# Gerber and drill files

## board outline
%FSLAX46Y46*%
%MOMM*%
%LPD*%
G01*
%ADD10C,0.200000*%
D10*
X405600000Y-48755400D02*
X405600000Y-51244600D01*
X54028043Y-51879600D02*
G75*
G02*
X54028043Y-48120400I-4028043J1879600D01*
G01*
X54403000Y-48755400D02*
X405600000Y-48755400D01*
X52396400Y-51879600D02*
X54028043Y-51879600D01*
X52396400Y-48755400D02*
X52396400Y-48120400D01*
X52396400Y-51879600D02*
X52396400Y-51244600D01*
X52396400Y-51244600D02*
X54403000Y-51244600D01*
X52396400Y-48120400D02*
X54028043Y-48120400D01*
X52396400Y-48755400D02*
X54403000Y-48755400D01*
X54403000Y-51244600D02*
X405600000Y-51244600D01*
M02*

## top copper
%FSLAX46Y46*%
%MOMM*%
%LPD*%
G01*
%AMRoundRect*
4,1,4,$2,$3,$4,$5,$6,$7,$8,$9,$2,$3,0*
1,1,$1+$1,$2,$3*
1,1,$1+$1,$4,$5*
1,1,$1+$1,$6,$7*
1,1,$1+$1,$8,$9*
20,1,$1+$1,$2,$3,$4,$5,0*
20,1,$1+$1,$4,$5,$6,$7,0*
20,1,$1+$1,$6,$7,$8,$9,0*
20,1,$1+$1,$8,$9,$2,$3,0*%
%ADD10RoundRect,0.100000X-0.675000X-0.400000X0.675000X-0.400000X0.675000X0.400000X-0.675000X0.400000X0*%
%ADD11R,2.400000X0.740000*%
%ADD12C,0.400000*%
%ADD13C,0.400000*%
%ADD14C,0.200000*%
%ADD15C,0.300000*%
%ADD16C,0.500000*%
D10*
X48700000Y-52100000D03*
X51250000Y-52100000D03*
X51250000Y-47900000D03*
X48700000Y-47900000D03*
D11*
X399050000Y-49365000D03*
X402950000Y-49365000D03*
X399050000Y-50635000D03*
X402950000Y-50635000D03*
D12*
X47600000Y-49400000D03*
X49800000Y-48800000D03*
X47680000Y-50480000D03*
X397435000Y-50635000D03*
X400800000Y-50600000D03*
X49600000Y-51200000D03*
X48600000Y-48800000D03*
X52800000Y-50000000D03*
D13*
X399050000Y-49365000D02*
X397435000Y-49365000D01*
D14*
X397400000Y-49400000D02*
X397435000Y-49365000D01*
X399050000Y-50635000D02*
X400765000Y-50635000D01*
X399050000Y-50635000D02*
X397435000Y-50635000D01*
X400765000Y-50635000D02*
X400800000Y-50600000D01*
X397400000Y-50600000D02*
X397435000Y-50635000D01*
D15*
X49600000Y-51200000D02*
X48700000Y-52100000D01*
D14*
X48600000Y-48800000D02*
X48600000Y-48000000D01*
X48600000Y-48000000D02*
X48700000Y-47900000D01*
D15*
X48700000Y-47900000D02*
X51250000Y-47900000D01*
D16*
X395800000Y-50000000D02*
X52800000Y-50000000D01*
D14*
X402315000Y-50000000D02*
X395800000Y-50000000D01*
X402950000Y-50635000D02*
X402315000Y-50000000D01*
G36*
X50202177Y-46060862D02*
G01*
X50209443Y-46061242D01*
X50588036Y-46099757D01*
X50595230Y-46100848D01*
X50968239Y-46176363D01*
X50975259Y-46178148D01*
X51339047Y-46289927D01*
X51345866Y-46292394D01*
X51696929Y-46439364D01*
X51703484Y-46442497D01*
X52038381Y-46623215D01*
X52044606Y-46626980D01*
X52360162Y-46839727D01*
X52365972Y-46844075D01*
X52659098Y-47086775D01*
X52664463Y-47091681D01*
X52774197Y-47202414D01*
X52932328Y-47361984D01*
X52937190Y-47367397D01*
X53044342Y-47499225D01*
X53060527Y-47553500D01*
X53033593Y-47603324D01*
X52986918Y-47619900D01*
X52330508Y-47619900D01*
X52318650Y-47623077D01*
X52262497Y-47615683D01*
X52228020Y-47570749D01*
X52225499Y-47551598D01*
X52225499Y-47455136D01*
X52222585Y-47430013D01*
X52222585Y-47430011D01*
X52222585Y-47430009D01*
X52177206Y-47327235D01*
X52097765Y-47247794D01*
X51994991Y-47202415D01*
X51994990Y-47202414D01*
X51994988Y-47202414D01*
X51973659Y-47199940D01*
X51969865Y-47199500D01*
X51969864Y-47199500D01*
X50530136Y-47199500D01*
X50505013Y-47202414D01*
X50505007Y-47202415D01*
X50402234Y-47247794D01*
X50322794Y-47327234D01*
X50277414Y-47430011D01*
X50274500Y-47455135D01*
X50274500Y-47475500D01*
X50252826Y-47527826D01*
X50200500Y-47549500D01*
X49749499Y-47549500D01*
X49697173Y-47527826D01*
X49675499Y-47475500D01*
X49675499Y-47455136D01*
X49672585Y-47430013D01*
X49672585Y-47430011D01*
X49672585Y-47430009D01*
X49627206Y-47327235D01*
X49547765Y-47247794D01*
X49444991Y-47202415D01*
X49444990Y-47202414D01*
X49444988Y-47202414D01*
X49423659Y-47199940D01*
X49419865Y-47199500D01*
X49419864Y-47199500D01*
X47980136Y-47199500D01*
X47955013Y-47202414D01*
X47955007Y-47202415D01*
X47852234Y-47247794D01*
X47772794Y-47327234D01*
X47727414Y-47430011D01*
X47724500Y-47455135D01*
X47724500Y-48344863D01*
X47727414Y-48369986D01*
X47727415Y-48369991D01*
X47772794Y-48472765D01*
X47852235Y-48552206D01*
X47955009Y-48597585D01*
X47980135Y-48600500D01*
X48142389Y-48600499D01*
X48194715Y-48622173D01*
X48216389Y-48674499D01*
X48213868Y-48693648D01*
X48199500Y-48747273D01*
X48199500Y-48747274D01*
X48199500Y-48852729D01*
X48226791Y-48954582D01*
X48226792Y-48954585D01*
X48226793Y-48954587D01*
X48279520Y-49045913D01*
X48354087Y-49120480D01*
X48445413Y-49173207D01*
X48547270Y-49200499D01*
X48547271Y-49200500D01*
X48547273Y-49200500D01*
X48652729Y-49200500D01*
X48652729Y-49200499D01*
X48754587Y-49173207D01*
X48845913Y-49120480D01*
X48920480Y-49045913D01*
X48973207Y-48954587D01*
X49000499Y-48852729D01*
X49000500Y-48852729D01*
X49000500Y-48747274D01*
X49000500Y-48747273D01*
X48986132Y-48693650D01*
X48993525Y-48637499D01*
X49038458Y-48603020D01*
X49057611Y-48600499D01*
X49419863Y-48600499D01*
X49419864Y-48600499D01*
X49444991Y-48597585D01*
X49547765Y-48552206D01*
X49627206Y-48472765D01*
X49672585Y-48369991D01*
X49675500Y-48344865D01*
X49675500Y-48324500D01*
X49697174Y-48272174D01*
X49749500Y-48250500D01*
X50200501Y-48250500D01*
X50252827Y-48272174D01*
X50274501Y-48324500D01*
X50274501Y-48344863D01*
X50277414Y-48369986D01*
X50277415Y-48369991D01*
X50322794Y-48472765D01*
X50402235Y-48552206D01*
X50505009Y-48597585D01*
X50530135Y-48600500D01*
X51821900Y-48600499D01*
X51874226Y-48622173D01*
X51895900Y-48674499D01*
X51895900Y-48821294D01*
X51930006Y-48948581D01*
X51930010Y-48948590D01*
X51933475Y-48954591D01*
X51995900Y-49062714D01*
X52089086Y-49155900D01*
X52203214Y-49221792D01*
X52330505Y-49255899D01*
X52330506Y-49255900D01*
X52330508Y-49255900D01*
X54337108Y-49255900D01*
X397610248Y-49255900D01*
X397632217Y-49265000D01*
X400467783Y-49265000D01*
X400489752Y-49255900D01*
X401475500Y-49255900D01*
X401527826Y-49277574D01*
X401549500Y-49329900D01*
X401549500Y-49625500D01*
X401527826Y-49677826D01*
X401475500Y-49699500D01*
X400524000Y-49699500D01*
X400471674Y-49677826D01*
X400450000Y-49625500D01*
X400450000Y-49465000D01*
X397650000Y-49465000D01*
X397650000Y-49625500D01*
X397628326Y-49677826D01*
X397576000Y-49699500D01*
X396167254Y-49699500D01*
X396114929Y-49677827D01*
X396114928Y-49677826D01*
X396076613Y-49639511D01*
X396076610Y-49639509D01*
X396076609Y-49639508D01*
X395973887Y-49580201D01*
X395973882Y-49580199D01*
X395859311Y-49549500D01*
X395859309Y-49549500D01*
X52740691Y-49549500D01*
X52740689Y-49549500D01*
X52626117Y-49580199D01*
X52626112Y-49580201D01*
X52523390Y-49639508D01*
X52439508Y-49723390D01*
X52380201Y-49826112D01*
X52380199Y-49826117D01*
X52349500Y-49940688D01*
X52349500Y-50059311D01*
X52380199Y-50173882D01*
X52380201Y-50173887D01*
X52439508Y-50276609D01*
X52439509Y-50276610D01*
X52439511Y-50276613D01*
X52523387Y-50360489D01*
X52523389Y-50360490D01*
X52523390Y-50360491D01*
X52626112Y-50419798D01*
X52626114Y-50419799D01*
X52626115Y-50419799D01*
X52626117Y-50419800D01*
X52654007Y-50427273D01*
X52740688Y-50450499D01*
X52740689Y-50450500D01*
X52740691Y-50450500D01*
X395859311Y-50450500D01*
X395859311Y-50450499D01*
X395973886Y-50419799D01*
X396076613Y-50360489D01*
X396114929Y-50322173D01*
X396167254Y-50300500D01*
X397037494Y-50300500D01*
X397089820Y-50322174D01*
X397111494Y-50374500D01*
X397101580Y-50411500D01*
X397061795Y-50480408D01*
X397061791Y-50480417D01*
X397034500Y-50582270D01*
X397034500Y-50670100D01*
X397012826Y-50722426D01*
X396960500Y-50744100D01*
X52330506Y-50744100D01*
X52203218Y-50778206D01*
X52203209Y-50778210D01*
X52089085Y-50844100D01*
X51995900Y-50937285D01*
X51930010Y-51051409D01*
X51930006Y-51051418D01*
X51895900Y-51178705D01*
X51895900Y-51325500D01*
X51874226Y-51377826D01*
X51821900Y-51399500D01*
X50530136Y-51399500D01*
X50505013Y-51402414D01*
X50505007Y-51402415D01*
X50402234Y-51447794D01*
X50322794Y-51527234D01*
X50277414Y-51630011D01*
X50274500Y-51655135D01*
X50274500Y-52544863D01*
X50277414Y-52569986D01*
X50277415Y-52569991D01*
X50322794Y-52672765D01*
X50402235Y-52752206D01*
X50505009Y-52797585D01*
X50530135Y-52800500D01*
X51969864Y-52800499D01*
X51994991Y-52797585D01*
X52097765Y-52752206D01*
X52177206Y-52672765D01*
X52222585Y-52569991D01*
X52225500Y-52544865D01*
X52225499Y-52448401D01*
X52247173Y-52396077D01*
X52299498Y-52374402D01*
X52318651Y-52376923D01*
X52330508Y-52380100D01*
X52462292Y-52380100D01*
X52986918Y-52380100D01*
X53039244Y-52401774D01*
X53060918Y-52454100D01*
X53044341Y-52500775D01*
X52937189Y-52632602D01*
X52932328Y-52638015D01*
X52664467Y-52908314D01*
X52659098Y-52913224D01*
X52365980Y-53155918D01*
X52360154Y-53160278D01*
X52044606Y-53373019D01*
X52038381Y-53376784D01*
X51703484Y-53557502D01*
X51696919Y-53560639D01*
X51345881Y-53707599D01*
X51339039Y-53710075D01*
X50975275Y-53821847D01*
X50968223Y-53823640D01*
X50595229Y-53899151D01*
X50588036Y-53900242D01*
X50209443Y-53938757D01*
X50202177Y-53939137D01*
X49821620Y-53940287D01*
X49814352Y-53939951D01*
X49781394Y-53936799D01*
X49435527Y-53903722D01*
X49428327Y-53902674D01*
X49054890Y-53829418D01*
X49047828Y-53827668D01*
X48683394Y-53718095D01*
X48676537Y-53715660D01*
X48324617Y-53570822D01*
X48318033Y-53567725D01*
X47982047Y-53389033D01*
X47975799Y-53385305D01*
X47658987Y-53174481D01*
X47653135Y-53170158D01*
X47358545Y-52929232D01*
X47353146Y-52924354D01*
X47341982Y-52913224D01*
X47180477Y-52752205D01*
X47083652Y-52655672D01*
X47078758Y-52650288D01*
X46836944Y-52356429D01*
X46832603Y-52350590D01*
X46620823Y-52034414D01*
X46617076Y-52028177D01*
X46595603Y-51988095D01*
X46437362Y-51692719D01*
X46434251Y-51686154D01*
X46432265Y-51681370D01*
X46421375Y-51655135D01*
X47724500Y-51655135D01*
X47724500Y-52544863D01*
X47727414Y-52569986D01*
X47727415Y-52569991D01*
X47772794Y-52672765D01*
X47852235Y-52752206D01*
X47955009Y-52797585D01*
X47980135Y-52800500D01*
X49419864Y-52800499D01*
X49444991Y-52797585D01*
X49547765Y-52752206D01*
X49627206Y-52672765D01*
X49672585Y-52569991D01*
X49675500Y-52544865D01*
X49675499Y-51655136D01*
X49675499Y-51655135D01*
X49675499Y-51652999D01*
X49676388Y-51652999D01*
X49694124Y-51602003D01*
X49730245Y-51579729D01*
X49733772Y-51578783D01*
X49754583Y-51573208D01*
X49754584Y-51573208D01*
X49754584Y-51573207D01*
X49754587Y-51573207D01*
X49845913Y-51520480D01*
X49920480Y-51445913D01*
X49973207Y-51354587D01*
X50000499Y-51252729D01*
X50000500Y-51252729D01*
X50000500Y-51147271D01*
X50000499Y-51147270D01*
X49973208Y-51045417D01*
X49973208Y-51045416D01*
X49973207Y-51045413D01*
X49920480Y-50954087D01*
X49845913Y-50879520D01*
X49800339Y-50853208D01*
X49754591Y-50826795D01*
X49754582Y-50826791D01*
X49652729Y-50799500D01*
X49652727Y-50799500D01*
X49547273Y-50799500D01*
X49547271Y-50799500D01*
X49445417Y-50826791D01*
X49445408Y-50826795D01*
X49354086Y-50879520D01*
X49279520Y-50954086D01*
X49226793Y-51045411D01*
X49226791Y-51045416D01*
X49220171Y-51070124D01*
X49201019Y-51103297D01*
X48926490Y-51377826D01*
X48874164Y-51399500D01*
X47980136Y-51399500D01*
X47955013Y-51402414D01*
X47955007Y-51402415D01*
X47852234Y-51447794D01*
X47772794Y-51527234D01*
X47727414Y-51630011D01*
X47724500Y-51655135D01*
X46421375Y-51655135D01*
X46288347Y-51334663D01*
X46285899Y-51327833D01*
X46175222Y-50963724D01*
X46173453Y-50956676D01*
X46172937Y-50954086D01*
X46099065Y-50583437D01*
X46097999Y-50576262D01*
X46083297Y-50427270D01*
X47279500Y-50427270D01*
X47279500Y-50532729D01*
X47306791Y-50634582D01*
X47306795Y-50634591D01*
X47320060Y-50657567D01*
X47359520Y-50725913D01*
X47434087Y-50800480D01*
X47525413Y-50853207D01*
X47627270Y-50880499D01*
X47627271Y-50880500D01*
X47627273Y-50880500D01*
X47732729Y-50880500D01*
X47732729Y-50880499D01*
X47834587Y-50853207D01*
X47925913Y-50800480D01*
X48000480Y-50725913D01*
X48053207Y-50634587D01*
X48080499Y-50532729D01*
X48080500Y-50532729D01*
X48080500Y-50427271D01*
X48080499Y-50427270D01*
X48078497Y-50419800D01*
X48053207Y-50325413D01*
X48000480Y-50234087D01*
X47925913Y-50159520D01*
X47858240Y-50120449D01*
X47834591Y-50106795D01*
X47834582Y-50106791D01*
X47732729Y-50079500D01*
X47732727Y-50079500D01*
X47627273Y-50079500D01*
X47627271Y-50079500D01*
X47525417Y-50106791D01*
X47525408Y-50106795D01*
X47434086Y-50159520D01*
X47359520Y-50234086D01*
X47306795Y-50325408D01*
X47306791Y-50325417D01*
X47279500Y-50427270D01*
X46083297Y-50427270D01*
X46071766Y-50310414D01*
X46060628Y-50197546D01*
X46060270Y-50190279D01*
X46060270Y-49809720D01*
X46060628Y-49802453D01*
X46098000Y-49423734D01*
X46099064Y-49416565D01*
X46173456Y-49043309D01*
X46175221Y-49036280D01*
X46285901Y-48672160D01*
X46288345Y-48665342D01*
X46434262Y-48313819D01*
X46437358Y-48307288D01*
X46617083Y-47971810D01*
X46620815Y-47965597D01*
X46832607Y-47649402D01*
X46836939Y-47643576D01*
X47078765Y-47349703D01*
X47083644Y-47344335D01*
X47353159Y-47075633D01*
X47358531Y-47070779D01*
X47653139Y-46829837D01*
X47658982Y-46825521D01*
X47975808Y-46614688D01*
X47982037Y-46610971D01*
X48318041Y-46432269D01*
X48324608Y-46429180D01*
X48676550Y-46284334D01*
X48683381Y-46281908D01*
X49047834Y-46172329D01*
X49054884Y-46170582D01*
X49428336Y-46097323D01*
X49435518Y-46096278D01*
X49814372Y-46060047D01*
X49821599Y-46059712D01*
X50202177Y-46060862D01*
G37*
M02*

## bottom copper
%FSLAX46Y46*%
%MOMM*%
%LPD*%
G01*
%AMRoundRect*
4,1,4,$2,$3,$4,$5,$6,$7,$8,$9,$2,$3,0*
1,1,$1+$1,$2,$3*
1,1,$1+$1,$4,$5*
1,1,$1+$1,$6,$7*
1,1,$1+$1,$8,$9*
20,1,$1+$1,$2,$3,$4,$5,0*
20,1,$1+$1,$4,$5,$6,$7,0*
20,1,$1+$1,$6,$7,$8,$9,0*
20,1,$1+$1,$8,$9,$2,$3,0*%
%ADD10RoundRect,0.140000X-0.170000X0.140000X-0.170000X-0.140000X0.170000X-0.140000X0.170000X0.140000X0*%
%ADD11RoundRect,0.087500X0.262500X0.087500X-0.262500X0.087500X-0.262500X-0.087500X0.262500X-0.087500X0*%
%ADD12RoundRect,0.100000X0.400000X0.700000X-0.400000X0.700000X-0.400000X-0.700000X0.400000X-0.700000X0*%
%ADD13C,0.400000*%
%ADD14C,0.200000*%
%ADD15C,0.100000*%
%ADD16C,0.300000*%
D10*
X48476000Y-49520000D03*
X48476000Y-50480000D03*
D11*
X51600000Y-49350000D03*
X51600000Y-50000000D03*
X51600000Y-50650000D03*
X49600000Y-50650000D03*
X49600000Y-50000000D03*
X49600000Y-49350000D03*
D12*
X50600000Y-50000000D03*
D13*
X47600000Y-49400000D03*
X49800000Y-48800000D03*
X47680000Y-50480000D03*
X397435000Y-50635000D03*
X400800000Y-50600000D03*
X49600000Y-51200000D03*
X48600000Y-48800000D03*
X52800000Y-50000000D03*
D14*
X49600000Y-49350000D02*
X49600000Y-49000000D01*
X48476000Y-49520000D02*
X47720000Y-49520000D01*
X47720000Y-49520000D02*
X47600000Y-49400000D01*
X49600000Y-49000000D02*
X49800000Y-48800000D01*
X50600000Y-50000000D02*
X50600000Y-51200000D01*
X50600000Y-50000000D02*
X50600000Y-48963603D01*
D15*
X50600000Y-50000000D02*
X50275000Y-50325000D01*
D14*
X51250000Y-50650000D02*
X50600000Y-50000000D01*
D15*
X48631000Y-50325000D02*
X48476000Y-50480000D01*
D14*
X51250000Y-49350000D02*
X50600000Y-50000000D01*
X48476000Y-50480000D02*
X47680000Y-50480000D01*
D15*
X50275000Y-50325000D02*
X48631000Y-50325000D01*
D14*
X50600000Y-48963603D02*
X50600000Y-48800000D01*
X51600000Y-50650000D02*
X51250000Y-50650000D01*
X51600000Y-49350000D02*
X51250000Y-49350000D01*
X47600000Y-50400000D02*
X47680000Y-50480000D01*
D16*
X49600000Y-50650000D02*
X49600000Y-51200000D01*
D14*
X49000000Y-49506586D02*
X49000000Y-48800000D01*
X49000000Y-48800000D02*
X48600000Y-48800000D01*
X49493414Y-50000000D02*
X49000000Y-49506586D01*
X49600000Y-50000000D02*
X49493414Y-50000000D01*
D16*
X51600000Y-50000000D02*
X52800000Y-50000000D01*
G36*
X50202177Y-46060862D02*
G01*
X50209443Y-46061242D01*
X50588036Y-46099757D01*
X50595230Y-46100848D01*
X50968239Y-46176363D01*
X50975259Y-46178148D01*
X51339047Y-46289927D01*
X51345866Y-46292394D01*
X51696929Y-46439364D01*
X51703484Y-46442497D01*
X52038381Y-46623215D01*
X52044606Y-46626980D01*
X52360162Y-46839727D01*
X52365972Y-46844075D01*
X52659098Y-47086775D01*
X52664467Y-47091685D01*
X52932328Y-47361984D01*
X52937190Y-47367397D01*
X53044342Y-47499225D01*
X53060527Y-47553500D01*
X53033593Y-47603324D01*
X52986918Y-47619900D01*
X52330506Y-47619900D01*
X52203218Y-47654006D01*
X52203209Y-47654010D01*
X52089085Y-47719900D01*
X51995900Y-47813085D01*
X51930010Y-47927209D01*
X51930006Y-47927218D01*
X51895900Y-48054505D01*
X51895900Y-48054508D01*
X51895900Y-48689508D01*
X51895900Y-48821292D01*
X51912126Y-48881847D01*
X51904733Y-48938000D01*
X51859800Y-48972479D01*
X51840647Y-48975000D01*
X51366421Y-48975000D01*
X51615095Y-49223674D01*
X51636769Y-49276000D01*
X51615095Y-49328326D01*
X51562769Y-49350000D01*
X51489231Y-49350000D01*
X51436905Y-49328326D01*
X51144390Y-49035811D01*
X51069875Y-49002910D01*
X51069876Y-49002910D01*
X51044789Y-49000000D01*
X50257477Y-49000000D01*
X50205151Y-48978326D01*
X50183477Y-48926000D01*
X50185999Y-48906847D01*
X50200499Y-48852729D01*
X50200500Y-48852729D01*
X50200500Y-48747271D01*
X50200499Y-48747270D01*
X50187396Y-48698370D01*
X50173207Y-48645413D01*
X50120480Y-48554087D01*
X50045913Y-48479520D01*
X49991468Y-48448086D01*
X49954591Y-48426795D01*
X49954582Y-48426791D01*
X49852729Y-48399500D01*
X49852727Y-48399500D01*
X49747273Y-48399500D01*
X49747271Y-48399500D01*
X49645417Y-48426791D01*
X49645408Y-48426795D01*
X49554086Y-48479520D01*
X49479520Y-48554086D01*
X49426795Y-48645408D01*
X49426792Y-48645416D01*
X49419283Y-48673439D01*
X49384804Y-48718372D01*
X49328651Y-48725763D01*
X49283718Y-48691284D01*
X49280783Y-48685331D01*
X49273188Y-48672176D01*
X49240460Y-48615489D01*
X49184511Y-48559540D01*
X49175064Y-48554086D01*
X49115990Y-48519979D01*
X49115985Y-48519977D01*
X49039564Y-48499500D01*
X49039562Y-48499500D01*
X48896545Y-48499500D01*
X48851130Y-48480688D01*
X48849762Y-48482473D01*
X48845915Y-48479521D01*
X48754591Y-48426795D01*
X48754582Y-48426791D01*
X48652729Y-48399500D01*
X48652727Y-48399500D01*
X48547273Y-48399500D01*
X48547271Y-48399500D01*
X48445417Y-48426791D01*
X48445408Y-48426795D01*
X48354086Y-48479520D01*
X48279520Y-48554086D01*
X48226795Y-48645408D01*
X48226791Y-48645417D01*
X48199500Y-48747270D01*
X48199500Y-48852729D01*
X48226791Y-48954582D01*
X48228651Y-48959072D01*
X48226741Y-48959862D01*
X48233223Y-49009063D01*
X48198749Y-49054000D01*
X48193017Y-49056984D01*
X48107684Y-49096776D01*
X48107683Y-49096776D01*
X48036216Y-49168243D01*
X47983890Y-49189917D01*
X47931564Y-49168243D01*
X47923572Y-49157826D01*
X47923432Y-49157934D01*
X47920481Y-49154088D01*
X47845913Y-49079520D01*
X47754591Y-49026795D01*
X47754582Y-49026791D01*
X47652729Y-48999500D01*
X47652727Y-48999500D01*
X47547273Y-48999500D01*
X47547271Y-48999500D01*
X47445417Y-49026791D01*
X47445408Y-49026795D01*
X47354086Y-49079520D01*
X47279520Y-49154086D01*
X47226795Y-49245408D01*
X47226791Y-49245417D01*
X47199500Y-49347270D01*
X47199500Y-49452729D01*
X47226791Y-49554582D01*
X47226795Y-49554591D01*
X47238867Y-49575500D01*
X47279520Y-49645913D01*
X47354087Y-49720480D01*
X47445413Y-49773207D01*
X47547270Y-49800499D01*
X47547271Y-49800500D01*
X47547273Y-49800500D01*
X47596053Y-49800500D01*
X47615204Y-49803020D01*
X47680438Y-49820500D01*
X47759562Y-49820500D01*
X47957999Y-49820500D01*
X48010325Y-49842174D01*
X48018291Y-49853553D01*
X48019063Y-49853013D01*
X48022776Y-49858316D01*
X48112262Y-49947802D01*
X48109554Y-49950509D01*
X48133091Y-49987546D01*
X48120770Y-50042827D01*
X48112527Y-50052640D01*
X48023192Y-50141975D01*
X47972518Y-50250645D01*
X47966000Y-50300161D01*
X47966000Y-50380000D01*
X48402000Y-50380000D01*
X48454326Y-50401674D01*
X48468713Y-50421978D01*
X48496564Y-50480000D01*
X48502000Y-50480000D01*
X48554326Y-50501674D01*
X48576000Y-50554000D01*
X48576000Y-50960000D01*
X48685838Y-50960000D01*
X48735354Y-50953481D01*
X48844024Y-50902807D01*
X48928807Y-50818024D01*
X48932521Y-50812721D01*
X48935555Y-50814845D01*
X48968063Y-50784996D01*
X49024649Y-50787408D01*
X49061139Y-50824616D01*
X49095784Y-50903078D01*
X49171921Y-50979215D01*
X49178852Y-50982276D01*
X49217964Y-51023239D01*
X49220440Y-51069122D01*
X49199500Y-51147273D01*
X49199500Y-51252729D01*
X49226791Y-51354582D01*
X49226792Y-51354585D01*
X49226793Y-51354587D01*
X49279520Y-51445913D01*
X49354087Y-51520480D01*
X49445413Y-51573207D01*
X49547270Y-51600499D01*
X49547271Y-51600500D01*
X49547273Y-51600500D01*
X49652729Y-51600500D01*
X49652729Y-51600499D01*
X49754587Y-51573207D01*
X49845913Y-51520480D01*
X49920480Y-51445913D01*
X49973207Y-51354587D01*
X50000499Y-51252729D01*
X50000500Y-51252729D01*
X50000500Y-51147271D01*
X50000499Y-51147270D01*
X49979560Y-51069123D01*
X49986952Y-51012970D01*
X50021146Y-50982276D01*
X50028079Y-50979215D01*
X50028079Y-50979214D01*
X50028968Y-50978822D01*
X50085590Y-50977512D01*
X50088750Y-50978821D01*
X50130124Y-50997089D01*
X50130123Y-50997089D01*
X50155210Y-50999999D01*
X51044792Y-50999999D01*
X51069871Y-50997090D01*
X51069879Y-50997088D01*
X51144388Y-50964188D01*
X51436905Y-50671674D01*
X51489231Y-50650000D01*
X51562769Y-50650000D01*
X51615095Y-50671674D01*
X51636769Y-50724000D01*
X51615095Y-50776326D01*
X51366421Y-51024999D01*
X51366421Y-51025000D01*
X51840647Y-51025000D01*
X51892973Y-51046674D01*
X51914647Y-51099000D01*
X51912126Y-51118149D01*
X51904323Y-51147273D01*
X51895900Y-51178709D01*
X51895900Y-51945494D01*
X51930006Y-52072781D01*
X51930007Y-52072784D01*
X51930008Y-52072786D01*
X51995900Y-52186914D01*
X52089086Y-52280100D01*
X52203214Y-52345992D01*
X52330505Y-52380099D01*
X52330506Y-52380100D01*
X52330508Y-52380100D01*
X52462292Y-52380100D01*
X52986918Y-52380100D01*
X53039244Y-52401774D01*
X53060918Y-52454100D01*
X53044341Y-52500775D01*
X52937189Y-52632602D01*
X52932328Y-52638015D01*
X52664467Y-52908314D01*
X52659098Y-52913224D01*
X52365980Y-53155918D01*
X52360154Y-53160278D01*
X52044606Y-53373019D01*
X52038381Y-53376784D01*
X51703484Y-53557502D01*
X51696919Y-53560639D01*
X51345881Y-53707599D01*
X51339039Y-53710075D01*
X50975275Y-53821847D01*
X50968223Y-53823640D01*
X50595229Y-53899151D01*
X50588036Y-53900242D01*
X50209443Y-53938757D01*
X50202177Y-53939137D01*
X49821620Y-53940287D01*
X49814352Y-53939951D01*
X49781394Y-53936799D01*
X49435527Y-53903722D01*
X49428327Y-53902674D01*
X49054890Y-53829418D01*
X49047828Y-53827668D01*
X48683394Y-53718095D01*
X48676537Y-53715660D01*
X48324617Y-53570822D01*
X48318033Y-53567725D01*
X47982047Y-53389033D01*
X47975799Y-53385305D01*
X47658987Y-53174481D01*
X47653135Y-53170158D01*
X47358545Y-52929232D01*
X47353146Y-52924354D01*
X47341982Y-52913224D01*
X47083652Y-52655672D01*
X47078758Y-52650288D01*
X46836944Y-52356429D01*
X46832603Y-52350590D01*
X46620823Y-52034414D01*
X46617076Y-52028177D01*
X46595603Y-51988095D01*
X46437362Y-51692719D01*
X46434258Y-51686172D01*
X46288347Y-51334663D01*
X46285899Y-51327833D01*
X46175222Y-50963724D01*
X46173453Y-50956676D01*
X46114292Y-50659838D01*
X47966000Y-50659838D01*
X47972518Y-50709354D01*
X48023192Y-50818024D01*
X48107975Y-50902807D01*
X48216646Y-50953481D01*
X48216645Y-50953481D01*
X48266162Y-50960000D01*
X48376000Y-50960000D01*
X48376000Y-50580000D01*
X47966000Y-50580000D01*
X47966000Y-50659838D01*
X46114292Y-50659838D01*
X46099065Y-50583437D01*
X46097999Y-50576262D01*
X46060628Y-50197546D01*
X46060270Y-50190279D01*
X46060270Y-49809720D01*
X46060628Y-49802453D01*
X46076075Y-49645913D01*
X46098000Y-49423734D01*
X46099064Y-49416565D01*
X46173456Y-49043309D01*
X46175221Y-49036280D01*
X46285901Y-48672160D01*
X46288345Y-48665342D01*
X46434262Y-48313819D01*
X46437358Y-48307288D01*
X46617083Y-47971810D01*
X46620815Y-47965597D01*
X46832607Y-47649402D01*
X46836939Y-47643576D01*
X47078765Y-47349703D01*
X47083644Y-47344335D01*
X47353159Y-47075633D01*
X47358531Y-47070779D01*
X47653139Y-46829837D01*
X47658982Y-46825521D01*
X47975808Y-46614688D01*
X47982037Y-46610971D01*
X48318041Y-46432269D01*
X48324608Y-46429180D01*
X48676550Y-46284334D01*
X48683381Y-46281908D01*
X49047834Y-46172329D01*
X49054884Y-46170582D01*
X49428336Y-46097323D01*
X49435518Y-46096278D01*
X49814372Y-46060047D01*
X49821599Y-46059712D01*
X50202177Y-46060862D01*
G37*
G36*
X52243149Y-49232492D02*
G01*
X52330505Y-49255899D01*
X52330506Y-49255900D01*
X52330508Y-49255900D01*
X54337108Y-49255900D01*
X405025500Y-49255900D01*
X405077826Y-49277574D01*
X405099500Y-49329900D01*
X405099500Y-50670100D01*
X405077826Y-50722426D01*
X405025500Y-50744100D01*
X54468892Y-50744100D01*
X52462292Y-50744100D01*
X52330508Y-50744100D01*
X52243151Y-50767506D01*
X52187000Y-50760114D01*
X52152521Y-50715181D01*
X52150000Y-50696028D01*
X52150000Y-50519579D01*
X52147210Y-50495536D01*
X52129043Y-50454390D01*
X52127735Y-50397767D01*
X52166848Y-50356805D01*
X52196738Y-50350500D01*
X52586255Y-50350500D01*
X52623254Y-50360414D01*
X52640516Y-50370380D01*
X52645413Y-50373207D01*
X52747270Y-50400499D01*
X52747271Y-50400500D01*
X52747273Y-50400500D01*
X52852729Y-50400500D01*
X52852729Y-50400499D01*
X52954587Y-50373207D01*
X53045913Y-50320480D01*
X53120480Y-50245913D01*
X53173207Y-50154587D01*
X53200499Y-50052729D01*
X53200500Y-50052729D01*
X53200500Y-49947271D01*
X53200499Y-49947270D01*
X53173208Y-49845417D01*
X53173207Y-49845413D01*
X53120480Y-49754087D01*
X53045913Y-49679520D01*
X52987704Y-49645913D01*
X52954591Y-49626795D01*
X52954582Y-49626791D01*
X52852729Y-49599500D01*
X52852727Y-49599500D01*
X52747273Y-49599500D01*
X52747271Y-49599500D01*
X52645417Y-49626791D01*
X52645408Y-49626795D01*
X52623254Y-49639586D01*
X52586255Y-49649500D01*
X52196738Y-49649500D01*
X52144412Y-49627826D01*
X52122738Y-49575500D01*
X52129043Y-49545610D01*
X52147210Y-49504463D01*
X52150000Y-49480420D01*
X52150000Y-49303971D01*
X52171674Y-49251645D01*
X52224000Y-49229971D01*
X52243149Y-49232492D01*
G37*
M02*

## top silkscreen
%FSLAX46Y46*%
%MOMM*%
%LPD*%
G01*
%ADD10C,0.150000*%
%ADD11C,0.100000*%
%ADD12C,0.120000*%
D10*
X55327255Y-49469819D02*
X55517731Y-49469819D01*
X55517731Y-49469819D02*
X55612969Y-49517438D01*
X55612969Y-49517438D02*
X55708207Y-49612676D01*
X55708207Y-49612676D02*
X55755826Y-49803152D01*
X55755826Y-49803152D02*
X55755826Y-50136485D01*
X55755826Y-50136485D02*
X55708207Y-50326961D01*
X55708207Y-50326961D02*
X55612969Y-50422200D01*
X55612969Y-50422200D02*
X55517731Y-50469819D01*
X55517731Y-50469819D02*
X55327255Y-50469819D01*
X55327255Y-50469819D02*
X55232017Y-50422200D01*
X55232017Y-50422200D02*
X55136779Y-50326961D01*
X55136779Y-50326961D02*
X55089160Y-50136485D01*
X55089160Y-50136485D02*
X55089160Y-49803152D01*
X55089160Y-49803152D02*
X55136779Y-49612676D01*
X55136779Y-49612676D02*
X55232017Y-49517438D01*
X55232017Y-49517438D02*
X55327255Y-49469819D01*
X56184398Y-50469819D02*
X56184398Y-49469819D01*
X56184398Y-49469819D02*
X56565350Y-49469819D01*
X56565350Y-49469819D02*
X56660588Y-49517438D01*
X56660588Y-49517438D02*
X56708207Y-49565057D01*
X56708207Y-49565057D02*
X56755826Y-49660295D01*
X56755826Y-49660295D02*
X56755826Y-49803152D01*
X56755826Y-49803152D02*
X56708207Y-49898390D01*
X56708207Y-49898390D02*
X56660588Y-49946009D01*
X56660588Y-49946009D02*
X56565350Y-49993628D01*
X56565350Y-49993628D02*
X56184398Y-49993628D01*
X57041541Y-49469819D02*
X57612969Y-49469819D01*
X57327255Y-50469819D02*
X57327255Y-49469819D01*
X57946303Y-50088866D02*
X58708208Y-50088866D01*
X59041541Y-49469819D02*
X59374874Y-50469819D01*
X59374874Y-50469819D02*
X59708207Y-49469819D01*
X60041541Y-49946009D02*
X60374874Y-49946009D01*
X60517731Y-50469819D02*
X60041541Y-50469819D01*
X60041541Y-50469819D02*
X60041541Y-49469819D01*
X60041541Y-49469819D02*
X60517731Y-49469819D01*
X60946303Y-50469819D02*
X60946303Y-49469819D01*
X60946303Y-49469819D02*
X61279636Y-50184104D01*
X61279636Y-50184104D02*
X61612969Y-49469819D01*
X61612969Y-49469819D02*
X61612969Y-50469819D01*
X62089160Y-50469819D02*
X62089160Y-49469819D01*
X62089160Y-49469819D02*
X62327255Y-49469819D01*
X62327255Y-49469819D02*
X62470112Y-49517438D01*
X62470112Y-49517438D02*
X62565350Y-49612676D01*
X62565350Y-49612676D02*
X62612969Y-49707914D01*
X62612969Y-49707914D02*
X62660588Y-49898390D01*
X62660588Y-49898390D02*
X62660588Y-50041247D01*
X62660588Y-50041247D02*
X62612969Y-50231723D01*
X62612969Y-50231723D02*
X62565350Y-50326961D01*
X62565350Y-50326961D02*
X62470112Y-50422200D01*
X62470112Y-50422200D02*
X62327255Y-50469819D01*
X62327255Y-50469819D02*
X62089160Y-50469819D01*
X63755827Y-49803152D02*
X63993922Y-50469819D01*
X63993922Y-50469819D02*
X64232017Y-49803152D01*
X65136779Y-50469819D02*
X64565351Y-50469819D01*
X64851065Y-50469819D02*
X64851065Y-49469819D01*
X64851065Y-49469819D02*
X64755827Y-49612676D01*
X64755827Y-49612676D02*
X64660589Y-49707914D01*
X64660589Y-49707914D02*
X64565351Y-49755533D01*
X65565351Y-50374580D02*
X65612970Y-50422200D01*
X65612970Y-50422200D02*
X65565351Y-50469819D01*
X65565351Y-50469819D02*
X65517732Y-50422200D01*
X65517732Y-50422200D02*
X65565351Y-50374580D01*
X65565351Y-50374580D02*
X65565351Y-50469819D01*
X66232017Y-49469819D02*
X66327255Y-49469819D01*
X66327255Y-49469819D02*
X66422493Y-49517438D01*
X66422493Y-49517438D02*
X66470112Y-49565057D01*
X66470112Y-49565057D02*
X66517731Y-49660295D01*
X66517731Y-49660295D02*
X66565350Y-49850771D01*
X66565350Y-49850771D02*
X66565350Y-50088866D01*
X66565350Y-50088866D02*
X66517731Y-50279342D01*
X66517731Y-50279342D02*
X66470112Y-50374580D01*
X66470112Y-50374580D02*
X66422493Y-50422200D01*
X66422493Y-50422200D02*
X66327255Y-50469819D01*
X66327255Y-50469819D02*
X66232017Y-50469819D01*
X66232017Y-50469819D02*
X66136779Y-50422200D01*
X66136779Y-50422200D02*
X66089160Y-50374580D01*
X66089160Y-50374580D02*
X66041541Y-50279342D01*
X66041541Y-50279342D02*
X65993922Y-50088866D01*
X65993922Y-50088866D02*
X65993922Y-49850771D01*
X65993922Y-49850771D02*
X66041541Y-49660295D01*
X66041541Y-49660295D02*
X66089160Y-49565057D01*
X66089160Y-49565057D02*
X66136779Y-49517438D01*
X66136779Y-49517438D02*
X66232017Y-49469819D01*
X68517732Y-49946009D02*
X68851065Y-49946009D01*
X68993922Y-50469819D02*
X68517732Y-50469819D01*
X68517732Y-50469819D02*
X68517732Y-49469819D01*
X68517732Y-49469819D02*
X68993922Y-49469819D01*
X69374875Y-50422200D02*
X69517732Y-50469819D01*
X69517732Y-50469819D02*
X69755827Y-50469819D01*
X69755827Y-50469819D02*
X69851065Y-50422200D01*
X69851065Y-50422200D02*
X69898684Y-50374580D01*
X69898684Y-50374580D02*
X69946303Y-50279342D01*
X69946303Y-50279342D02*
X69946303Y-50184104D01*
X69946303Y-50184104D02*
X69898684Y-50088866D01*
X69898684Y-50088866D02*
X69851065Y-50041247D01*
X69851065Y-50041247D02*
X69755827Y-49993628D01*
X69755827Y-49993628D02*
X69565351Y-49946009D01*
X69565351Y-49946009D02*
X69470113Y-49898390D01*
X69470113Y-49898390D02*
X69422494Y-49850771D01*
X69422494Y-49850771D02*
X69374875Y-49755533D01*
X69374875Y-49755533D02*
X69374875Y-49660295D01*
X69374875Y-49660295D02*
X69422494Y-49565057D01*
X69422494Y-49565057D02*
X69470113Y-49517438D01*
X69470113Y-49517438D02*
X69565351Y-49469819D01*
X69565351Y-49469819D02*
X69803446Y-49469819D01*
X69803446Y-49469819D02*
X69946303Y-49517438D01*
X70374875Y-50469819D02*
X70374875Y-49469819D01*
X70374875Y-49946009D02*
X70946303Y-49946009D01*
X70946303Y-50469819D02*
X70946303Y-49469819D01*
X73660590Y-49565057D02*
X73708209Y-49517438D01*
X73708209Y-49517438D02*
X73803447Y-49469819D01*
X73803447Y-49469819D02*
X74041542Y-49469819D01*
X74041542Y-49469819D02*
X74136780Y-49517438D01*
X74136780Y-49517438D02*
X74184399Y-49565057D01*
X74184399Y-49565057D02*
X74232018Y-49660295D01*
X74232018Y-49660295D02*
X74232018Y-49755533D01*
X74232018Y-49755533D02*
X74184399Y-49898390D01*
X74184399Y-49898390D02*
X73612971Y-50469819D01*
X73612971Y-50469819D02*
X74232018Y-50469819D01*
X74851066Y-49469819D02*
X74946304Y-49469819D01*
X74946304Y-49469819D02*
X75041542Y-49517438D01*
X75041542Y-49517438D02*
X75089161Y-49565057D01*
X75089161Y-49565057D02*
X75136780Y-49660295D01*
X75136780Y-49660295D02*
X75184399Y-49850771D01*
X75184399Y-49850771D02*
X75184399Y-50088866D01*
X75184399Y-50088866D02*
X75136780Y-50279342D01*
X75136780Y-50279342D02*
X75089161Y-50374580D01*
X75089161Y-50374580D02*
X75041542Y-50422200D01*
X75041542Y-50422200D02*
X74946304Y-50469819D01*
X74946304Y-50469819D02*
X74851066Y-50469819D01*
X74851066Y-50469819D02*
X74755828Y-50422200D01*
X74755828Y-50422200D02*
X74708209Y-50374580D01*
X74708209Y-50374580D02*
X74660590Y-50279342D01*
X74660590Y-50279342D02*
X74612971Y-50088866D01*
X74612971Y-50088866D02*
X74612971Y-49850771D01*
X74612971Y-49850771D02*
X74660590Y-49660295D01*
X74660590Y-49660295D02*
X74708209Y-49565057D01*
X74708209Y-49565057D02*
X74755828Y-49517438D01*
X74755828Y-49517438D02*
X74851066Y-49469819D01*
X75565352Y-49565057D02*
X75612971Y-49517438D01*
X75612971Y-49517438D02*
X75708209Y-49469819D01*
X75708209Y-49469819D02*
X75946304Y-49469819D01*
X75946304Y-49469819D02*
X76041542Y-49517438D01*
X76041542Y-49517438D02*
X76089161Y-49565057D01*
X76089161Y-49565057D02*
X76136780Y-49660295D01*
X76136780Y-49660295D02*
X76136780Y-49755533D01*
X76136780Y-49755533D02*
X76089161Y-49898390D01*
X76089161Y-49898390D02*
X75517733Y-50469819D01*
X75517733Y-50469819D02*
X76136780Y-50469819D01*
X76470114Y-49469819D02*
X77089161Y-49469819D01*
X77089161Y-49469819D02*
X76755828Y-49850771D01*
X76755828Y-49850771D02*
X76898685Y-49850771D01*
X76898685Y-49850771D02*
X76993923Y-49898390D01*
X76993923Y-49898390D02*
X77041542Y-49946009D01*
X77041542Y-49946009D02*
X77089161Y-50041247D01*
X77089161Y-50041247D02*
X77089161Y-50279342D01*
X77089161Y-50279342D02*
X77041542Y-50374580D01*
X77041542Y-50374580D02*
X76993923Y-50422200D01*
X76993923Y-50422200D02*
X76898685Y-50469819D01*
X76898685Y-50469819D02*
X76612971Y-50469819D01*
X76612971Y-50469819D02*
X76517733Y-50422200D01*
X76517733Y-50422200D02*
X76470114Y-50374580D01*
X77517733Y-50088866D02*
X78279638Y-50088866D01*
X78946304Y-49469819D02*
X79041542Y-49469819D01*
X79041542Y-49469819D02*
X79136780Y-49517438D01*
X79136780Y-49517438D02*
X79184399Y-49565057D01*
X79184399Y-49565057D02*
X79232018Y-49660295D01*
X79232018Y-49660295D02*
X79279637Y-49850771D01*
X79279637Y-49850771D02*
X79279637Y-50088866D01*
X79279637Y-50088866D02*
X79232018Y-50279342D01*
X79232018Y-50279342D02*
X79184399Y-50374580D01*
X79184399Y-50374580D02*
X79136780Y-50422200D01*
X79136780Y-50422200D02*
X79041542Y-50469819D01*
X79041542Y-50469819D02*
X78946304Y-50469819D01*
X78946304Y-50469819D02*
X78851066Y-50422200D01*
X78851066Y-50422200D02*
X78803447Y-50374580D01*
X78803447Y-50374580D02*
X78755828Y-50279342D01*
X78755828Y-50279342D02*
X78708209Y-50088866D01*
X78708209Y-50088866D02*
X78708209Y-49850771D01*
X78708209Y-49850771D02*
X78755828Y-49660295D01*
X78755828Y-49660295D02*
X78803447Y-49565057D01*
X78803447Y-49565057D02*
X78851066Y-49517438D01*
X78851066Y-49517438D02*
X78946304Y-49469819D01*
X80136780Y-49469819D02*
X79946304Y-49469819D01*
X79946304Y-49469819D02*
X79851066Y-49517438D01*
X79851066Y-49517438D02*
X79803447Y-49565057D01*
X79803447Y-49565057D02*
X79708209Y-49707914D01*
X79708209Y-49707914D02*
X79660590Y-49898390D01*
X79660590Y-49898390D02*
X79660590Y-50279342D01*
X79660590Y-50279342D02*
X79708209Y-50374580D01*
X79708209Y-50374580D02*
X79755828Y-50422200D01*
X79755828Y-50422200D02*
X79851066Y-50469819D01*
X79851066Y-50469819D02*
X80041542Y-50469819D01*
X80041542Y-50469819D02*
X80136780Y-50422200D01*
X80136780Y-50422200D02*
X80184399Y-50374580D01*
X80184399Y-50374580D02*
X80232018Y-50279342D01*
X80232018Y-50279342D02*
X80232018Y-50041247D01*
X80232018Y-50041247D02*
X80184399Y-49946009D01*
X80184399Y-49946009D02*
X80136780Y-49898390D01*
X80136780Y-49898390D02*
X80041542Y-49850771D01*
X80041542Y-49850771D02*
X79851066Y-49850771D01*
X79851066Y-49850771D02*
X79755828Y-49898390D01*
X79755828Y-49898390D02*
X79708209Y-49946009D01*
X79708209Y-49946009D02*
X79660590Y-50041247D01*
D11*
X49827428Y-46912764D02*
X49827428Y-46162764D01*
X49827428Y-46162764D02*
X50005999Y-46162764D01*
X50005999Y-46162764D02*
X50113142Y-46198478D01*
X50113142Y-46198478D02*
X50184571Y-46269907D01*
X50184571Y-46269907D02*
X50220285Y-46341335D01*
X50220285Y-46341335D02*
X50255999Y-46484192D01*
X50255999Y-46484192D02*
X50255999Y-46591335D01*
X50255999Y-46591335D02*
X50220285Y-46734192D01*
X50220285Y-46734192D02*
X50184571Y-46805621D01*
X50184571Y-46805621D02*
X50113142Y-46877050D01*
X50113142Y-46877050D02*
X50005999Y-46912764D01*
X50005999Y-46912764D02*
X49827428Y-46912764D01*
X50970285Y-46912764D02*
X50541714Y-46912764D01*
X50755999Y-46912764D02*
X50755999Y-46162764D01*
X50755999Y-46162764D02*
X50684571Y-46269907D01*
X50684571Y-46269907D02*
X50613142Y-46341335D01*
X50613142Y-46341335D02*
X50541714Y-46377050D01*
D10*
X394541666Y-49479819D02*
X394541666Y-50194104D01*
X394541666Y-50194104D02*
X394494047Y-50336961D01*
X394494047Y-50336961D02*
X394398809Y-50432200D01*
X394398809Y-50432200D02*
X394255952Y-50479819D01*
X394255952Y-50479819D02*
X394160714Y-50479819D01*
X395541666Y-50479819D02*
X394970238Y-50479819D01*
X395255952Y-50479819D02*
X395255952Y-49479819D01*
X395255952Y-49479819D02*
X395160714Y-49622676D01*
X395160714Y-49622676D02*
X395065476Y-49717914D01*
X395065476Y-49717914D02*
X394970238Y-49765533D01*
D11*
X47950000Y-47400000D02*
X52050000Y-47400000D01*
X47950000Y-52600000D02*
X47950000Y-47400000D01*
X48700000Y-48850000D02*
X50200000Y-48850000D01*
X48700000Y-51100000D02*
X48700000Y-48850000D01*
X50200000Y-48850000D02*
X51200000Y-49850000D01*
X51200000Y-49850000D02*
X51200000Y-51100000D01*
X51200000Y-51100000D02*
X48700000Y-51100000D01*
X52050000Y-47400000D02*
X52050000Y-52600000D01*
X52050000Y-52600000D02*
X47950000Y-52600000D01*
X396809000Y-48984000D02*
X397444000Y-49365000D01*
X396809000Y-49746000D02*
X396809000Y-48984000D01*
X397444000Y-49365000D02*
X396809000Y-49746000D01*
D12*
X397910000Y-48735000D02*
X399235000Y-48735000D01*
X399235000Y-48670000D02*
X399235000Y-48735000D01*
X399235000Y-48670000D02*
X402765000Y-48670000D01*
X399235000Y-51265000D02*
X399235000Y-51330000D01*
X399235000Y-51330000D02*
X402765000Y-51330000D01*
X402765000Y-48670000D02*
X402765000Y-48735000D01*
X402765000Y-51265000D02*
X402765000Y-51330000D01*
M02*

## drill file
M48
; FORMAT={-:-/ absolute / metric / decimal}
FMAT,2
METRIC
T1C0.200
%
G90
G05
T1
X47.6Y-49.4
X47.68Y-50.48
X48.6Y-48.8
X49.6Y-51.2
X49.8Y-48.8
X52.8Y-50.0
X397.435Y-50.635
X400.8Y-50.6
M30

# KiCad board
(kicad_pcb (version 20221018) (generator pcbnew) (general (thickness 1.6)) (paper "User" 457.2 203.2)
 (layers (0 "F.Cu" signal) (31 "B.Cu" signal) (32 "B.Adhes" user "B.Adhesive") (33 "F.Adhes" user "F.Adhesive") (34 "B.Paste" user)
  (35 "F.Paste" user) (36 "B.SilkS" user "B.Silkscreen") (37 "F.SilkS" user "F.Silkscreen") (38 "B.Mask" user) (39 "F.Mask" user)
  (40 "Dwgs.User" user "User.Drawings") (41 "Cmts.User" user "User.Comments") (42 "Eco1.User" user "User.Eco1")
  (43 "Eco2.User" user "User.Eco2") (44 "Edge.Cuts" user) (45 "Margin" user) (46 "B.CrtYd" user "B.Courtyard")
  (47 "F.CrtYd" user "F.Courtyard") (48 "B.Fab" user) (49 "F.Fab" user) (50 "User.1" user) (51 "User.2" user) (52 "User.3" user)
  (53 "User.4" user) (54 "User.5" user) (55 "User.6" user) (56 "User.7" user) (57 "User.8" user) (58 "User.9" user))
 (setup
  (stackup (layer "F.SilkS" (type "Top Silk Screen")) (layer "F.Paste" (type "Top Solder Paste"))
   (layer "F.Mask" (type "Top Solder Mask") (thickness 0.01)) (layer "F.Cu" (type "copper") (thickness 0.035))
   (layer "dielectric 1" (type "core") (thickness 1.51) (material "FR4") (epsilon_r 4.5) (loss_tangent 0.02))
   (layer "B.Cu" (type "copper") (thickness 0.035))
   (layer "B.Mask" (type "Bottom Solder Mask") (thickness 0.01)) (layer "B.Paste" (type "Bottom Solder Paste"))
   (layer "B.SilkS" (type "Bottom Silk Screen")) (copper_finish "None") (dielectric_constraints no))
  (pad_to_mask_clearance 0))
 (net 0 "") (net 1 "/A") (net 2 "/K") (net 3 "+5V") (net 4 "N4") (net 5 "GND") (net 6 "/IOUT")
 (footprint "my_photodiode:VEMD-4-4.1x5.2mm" (layer "F.Cu") (at 48.7 52.1)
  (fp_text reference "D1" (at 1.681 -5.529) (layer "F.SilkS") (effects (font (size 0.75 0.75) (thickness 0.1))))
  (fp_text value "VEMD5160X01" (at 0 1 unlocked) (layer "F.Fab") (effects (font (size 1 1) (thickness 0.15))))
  (fp_line (start -0.75 -4.7) (end 3.35 -4.7) (stroke (width 0.1) (type default)) (layer "F.SilkS"))
  (fp_line (start -0.75 0.5) (end -0.75 -4.7) (stroke (width 0.1) (type default)) (layer "F.SilkS"))
  (fp_line (start 0 -3.25) (end 1.5 -3.25) (stroke (width 0.1) (type default)) (layer "F.SilkS"))
  (fp_line (start 0 -1) (end 0 -3.25) (stroke (width 0.1) (type default)) (layer "F.SilkS"))
  (fp_line (start 1.5 -3.25) (end 2.5 -2.25) (stroke (width 0.1) (type default)) (layer "F.SilkS"))
  (fp_line (start 2.5 -2.25) (end 2.5 -1) (stroke (width 0.1) (type default)) (layer "F.SilkS"))
  (fp_line (start 2.5 -1) (end 0 -1) (stroke (width 0.1) (type default)) (layer "F.SilkS"))
  (fp_line (start 3.35 -4.7) (end 3.35 0.5) (stroke (width 0.1) (type default)) (layer "F.SilkS"))
  (fp_line (start 3.35 0.5) (end -0.75 0.5) (stroke (width 0.1) (type default)) (layer "F.SilkS"))
  (pad "1" smd roundrect (at 0 0) (size 1.55 1) (layers "F.Cu" "F.Paste" "F.Mask") (roundrect_rratio 0.1) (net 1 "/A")
   (thermal_bridge_angle 45))
  (pad "2" smd roundrect (at 2.55 0) (size 1.55 1) (layers "F.Cu" "F.Paste" "F.Mask") (roundrect_rratio 0.1) (thermal_bridge_angle 45))
  (pad "3" smd roundrect (at 2.55 -4.2) (size 1.55 1) (layers "F.Cu" "F.Paste" "F.Mask") (roundrect_rratio 0.1) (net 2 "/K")
   (thermal_bridge_angle 45))
  (pad "4" smd roundrect (at 0 -4.2) (size 1.55 1) (layers "F.Cu" "F.Paste" "F.Mask") (roundrect_rratio 0.1) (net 2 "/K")
   (thermal_bridge_angle 45)))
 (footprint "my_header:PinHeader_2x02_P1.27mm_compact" (layer "F.Cu") (at 401 50)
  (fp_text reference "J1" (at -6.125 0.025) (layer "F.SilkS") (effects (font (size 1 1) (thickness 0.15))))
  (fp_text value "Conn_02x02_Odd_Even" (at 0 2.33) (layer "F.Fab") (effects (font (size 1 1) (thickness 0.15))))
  (fp_line (start -4.191 -1.016) (end -3.556 -0.635) (stroke (width 0.1) (type default)) (layer "F.SilkS"))
  (fp_line (start -4.191 -0.254) (end -4.191 -1.016) (stroke (width 0.1) (type default)) (layer "F.SilkS"))
  (fp_line (start -3.556 -0.635) (end -4.191 -0.254) (stroke (width 0.1) (type default)) (layer "F.SilkS"))
  (fp_line (start -3.09 -1.265) (end -1.765 -1.265) (stroke (width 0.12) (type solid)) (layer "F.SilkS"))
  (fp_line (start -1.765 -1.33) (end -1.765 -1.265) (stroke (width 0.12) (type solid)) (layer "F.SilkS"))
  (fp_line (start -1.765 -1.33) (end 1.765 -1.33) (stroke (width 0.12) (type solid)) (layer "F.SilkS"))
  (fp_line (start -1.765 1.265) (end -1.765 1.33) (stroke (width 0.12) (type solid)) (layer "F.SilkS"))
  (fp_line (start -1.765 1.33) (end 1.765 1.33) (stroke (width 0.12) (type solid)) (layer "F.SilkS"))
  (fp_line (start 1.765 -1.33) (end 1.765 -1.265) (stroke (width 0.12) (type solid)) (layer "F.SilkS"))
  (fp_line (start 1.765 1.265) (end 1.765 1.33) (stroke (width 0.12) (type solid)) (layer "F.SilkS"))
  (pad "1" smd rect (at -1.95 -0.635) (size 2.4 0.74) (layers "F.Cu" "F.Paste" "F.Mask") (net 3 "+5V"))
  (pad "2" smd rect (at 1.95 -0.635) (size 2.4 0.74) (layers "F.Cu" "F.Paste" "F.Mask") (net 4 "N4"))
  (pad "3" smd rect (at -1.95 0.635) (size 2.4 0.74) (layers "F.Cu" "F.Paste" "F.Mask") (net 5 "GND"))
  (pad "4" smd rect (at 1.95 0.635) (size 2.4 0.74) (layers "F.Cu" "F.Paste" "F.Mask") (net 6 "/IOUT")))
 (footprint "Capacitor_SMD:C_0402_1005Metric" (layer "B.Cu") (at 48.476 50 -90)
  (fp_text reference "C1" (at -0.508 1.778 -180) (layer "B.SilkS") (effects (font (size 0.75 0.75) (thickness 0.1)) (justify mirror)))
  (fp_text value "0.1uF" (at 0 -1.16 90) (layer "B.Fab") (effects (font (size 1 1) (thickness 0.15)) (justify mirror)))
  (pad "1" smd roundrect (at -0.48 0 270) (size 0.56 0.62) (layers "B.Cu" "B.Paste" "B.Mask") (roundrect_rratio 0.25) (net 3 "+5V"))
  (pad "2" smd roundrect (at 0.48 0 270) (size 0.56 0.62) (layers "B.Cu" "B.Paste" "B.Mask") (roundrect_rratio 0.25) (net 5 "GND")))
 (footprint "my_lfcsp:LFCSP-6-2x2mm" (layer "B.Cu") (at 51.6 49.35 180)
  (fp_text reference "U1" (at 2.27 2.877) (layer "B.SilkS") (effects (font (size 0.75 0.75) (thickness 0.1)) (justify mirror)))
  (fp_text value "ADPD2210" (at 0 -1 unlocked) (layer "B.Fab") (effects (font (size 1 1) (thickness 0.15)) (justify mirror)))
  (pad "1" smd roundrect (at 0 0 180) (size 0.7 0.35) (layers "B.Cu" "B.Paste" "B.Mask") (roundrect_rratio 0.25) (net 5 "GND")
   (thermal_bridge_angle 45))
  (pad "2" smd roundrect (at 0 -0.65 180) (size 0.7 0.35) (layers "B.Cu" "B.Paste" "B.Mask") (roundrect_rratio 0.25) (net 6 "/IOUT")
   (thermal_bridge_angle 45))
  (pad "3" smd roundrect (at 0 -1.3 180) (size 0.7 0.35) (layers "B.Cu" "B.Paste" "B.Mask") (roundrect_rratio 0.25) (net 5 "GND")
   (thermal_bridge_angle 45))
  (pad "4" smd roundrect (at 2 -1.3 180) (size 0.7 0.35) (layers "B.Cu" "B.Paste" "B.Mask") (roundrect_rratio 0.25) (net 1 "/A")
   (thermal_bridge_angle 45))
  (pad "5" smd roundrect (at 2 -0.65 180) (size 0.7 0.35) (layers "B.Cu" "B.Paste" "B.Mask") (roundrect_rratio 0.25) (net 2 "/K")
   (thermal_bridge_angle 45))
  (pad "6" smd roundrect (at 2 0 180) (size 0.7 0.35) (layers "B.Cu" "B.Paste" "B.Mask") (roundrect_rratio 0.25) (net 3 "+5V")
   (thermal_bridge_angle 45))
  (pad "7" smd roundrect (at 1 -0.65 180) (size 1 1.6) (layers "B.Cu" "B.Paste" "B.Mask") (roundrect_rratio 0.1) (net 5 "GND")
   (thermal_bridge_angle 45)))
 (gr_line (start 405.6 48.7554) (end 405.6 51.2446) (stroke (width 0.2) (type solid)) (layer "Edge.Cuts"))
 (gr_arc (start 54.028043 51.8796) (mid 45.555 50) (end 54.028043 48.1204) (stroke (width 0.2) (type solid)) (layer "Edge.Cuts"))
 (gr_line (start 54.403 48.7554) (end 405.6 48.7554) (stroke (width 0.2) (type solid)) (layer "Edge.Cuts"))
 (gr_line (start 52.3964 51.8796) (end 54.028043 51.8796) (stroke (width 0.2) (type solid)) (layer "Edge.Cuts"))
 (gr_line (start 52.3964 48.7554) (end 52.3964 48.1204) (stroke (width 0.2) (type solid)) (layer "Edge.Cuts"))
 (gr_line (start 52.3964 51.8796) (end 52.3964 51.2446) (stroke (width 0.2) (type solid)) (layer "Edge.Cuts"))
 (gr_line (start 52.3964 51.2446) (end 54.403 51.2446) (stroke (width 0.2) (type solid)) (layer "Edge.Cuts"))
 (gr_line (start 52.3964 48.1204) (end 54.028043 48.1204) (stroke (width 0.2) (type solid)) (layer "Edge.Cuts"))
 (gr_line (start 52.3964 48.7554) (end 54.403 48.7554) (stroke (width 0.2) (type solid)) (layer "Edge.Cuts"))
 (gr_line (start 54.403 51.2446) (end 405.6 51.2446) (stroke (width 0.2) (type solid)) (layer "Edge.Cuts"))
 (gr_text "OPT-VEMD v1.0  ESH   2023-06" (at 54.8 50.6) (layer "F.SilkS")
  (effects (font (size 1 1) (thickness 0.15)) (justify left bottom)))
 (segment (start 399.05 49.365) (end 397.435 49.365) (width 0.4) (layer "F.Cu") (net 3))
 (segment (start 397.4 49.4) (end 397.435 49.365) (width 0.2) (layer "F.Cu") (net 3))
 (via (at 47.6 49.4) (size 0.4) (drill 0.2) (layers "F.Cu" "B.Cu") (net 3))
 (via (at 49.8 48.8) (size 0.4) (drill 0.2) (layers "F.Cu" "B.Cu") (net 3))
 (segment (start 49.6 49.35) (end 49.6 49) (width 0.2) (layer "B.Cu") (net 3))
 (segment (start 48.476 49.52) (end 47.72 49.52) (width 0.2) (layer "B.Cu") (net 3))
 (segment (start 47.72 49.52) (end 47.6 49.4) (width 0.2) (layer "B.Cu") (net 3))
 (segment (start 49.6 49) (end 49.8 48.8) (width 0.2) (layer "B.Cu") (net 3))
 (segment (start 399.05 50.635) (end 400.765 50.635) (width 0.2) (layer "F.Cu") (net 5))
 (segment (start 399.05 50.635) (end 397.435 50.635) (width 0.2) (layer "F.Cu") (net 5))
 (segment (start 400.765 50.635) (end 400.8 50.6) (width 0.2) (layer "F.Cu") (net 5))
 (segment (start 397.4 50.6) (end 397.435 50.635) (width 0.2) (layer "F.Cu") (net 5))
 (via (at 47.68 50.48) (size 0.4) (drill 0.2) (layers "F.Cu" "B.Cu") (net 5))
 (via (at 397.435 50.635) (size 0.4) (drill 0.2) (layers "F.Cu" "B.Cu") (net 5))
 (via (at 400.8 50.6) (size 0.4) (drill 0.2) (layers "F.Cu" "B.Cu") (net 5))
 (segment (start 50.6 50) (end 50.6 51.2) (width 0.2) (layer "B.Cu") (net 5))
 (segment (start 50.6 50) (end 50.6 48.963603) (width 0.2) (layer "B.Cu") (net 5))
 (segment (start 50.6 50) (end 50.275 50.325) (width 0.1) (layer "B.Cu") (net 5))
 (segment (start 51.25 50.65) (end 50.6 50) (width 0.2) (layer "B.Cu") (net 5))
 (segment (start 48.631 50.325) (end 48.476 50.48) (width 0.1) (layer "B.Cu") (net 5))
 (segment (start 51.25 49.35) (end 50.6 50) (width 0.2) (layer "B.Cu") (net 5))
 (segment (start 48.476 50.48) (end 47.68 50.48) (width 0.2) (layer "B.Cu") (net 5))
 (segment (start 50.275 50.325) (end 48.631 50.325) (width 0.1) (layer "B.Cu") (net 5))
 (segment (start 50.6 48.963603) (end 50.6 48.8) (width 0.2) (layer "B.Cu") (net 5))
 (segment (start 51.6 50.65) (end 51.25 50.65) (width 0.2) (layer "B.Cu") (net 5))
 (segment (start 51.6 49.35) (end 51.25 49.35) (width 0.2) (layer "B.Cu") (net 5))
 (segment (start 47.6 50.4) (end 47.68 50.48) (width 0.2) (layer "B.Cu") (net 5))
 (segment (start 49.6 51.2) (end 48.7 52.1) (width 0.3) (layer "F.Cu") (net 1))
 (via (at 49.6 51.2) (size 0.4) (drill 0.2) (layers "F.Cu" "B.Cu") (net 1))
 (segment (start 49.6 50.65) (end 49.6 51.2) (width 0.3) (layer "B.Cu") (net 1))
 (segment (start 48.6 48.8) (end 48.6 48) (width 0.2) (layer "F.Cu") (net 2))
 (segment (start 48.6 48) (end 48.7 47.9) (width 0.2) (layer "F.Cu") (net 2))
 (segment (start 48.7 47.9) (end 51.25 47.9) (width 0.3) (layer "F.Cu") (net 2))
 (via (at 48.6 48.8) (size 0.4) (drill 0.2) (layers "F.Cu" "B.Cu") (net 2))
 (segment (start 49 49.506586) (end 49 48.8) (width 0.2) (layer "B.Cu") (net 2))
 (segment (start 49 48.8) (end 48.6 48.8) (width 0.2) (layer "B.Cu") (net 2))
 (segment (start 49.493414 50) (end 49 49.506586) (width 0.2) (layer "B.Cu") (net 2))
 (segment (start 49.6 50) (end 49.493414 50) (width 0.2) (layer "B.Cu") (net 2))
 (segment (start 395.8 50) (end 52.8 50) (width 0.5) (layer "F.Cu") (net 6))
 (segment (start 402.315 50) (end 395.8 50) (width 0.2) (layer "F.Cu") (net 6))
 (segment (start 402.95 50.635) (end 402.315 50) (width 0.2) (layer "F.Cu") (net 6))
 (via (at 52.8 50) (size 0.4) (drill 0.2) (layers "F.Cu" "B.Cu") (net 6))
 (segment (start 51.6 50) (end 52.8 50) (width 0.3) (layer "B.Cu") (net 6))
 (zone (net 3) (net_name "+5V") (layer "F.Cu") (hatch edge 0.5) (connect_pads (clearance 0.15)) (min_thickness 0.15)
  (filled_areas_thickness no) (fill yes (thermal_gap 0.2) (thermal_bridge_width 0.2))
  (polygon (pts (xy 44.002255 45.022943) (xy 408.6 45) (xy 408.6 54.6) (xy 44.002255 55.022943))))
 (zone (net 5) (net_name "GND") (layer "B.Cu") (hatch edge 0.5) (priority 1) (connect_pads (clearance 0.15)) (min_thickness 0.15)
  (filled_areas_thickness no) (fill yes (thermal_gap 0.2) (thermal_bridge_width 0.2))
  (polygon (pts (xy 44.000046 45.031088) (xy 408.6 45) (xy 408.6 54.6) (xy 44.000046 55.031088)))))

